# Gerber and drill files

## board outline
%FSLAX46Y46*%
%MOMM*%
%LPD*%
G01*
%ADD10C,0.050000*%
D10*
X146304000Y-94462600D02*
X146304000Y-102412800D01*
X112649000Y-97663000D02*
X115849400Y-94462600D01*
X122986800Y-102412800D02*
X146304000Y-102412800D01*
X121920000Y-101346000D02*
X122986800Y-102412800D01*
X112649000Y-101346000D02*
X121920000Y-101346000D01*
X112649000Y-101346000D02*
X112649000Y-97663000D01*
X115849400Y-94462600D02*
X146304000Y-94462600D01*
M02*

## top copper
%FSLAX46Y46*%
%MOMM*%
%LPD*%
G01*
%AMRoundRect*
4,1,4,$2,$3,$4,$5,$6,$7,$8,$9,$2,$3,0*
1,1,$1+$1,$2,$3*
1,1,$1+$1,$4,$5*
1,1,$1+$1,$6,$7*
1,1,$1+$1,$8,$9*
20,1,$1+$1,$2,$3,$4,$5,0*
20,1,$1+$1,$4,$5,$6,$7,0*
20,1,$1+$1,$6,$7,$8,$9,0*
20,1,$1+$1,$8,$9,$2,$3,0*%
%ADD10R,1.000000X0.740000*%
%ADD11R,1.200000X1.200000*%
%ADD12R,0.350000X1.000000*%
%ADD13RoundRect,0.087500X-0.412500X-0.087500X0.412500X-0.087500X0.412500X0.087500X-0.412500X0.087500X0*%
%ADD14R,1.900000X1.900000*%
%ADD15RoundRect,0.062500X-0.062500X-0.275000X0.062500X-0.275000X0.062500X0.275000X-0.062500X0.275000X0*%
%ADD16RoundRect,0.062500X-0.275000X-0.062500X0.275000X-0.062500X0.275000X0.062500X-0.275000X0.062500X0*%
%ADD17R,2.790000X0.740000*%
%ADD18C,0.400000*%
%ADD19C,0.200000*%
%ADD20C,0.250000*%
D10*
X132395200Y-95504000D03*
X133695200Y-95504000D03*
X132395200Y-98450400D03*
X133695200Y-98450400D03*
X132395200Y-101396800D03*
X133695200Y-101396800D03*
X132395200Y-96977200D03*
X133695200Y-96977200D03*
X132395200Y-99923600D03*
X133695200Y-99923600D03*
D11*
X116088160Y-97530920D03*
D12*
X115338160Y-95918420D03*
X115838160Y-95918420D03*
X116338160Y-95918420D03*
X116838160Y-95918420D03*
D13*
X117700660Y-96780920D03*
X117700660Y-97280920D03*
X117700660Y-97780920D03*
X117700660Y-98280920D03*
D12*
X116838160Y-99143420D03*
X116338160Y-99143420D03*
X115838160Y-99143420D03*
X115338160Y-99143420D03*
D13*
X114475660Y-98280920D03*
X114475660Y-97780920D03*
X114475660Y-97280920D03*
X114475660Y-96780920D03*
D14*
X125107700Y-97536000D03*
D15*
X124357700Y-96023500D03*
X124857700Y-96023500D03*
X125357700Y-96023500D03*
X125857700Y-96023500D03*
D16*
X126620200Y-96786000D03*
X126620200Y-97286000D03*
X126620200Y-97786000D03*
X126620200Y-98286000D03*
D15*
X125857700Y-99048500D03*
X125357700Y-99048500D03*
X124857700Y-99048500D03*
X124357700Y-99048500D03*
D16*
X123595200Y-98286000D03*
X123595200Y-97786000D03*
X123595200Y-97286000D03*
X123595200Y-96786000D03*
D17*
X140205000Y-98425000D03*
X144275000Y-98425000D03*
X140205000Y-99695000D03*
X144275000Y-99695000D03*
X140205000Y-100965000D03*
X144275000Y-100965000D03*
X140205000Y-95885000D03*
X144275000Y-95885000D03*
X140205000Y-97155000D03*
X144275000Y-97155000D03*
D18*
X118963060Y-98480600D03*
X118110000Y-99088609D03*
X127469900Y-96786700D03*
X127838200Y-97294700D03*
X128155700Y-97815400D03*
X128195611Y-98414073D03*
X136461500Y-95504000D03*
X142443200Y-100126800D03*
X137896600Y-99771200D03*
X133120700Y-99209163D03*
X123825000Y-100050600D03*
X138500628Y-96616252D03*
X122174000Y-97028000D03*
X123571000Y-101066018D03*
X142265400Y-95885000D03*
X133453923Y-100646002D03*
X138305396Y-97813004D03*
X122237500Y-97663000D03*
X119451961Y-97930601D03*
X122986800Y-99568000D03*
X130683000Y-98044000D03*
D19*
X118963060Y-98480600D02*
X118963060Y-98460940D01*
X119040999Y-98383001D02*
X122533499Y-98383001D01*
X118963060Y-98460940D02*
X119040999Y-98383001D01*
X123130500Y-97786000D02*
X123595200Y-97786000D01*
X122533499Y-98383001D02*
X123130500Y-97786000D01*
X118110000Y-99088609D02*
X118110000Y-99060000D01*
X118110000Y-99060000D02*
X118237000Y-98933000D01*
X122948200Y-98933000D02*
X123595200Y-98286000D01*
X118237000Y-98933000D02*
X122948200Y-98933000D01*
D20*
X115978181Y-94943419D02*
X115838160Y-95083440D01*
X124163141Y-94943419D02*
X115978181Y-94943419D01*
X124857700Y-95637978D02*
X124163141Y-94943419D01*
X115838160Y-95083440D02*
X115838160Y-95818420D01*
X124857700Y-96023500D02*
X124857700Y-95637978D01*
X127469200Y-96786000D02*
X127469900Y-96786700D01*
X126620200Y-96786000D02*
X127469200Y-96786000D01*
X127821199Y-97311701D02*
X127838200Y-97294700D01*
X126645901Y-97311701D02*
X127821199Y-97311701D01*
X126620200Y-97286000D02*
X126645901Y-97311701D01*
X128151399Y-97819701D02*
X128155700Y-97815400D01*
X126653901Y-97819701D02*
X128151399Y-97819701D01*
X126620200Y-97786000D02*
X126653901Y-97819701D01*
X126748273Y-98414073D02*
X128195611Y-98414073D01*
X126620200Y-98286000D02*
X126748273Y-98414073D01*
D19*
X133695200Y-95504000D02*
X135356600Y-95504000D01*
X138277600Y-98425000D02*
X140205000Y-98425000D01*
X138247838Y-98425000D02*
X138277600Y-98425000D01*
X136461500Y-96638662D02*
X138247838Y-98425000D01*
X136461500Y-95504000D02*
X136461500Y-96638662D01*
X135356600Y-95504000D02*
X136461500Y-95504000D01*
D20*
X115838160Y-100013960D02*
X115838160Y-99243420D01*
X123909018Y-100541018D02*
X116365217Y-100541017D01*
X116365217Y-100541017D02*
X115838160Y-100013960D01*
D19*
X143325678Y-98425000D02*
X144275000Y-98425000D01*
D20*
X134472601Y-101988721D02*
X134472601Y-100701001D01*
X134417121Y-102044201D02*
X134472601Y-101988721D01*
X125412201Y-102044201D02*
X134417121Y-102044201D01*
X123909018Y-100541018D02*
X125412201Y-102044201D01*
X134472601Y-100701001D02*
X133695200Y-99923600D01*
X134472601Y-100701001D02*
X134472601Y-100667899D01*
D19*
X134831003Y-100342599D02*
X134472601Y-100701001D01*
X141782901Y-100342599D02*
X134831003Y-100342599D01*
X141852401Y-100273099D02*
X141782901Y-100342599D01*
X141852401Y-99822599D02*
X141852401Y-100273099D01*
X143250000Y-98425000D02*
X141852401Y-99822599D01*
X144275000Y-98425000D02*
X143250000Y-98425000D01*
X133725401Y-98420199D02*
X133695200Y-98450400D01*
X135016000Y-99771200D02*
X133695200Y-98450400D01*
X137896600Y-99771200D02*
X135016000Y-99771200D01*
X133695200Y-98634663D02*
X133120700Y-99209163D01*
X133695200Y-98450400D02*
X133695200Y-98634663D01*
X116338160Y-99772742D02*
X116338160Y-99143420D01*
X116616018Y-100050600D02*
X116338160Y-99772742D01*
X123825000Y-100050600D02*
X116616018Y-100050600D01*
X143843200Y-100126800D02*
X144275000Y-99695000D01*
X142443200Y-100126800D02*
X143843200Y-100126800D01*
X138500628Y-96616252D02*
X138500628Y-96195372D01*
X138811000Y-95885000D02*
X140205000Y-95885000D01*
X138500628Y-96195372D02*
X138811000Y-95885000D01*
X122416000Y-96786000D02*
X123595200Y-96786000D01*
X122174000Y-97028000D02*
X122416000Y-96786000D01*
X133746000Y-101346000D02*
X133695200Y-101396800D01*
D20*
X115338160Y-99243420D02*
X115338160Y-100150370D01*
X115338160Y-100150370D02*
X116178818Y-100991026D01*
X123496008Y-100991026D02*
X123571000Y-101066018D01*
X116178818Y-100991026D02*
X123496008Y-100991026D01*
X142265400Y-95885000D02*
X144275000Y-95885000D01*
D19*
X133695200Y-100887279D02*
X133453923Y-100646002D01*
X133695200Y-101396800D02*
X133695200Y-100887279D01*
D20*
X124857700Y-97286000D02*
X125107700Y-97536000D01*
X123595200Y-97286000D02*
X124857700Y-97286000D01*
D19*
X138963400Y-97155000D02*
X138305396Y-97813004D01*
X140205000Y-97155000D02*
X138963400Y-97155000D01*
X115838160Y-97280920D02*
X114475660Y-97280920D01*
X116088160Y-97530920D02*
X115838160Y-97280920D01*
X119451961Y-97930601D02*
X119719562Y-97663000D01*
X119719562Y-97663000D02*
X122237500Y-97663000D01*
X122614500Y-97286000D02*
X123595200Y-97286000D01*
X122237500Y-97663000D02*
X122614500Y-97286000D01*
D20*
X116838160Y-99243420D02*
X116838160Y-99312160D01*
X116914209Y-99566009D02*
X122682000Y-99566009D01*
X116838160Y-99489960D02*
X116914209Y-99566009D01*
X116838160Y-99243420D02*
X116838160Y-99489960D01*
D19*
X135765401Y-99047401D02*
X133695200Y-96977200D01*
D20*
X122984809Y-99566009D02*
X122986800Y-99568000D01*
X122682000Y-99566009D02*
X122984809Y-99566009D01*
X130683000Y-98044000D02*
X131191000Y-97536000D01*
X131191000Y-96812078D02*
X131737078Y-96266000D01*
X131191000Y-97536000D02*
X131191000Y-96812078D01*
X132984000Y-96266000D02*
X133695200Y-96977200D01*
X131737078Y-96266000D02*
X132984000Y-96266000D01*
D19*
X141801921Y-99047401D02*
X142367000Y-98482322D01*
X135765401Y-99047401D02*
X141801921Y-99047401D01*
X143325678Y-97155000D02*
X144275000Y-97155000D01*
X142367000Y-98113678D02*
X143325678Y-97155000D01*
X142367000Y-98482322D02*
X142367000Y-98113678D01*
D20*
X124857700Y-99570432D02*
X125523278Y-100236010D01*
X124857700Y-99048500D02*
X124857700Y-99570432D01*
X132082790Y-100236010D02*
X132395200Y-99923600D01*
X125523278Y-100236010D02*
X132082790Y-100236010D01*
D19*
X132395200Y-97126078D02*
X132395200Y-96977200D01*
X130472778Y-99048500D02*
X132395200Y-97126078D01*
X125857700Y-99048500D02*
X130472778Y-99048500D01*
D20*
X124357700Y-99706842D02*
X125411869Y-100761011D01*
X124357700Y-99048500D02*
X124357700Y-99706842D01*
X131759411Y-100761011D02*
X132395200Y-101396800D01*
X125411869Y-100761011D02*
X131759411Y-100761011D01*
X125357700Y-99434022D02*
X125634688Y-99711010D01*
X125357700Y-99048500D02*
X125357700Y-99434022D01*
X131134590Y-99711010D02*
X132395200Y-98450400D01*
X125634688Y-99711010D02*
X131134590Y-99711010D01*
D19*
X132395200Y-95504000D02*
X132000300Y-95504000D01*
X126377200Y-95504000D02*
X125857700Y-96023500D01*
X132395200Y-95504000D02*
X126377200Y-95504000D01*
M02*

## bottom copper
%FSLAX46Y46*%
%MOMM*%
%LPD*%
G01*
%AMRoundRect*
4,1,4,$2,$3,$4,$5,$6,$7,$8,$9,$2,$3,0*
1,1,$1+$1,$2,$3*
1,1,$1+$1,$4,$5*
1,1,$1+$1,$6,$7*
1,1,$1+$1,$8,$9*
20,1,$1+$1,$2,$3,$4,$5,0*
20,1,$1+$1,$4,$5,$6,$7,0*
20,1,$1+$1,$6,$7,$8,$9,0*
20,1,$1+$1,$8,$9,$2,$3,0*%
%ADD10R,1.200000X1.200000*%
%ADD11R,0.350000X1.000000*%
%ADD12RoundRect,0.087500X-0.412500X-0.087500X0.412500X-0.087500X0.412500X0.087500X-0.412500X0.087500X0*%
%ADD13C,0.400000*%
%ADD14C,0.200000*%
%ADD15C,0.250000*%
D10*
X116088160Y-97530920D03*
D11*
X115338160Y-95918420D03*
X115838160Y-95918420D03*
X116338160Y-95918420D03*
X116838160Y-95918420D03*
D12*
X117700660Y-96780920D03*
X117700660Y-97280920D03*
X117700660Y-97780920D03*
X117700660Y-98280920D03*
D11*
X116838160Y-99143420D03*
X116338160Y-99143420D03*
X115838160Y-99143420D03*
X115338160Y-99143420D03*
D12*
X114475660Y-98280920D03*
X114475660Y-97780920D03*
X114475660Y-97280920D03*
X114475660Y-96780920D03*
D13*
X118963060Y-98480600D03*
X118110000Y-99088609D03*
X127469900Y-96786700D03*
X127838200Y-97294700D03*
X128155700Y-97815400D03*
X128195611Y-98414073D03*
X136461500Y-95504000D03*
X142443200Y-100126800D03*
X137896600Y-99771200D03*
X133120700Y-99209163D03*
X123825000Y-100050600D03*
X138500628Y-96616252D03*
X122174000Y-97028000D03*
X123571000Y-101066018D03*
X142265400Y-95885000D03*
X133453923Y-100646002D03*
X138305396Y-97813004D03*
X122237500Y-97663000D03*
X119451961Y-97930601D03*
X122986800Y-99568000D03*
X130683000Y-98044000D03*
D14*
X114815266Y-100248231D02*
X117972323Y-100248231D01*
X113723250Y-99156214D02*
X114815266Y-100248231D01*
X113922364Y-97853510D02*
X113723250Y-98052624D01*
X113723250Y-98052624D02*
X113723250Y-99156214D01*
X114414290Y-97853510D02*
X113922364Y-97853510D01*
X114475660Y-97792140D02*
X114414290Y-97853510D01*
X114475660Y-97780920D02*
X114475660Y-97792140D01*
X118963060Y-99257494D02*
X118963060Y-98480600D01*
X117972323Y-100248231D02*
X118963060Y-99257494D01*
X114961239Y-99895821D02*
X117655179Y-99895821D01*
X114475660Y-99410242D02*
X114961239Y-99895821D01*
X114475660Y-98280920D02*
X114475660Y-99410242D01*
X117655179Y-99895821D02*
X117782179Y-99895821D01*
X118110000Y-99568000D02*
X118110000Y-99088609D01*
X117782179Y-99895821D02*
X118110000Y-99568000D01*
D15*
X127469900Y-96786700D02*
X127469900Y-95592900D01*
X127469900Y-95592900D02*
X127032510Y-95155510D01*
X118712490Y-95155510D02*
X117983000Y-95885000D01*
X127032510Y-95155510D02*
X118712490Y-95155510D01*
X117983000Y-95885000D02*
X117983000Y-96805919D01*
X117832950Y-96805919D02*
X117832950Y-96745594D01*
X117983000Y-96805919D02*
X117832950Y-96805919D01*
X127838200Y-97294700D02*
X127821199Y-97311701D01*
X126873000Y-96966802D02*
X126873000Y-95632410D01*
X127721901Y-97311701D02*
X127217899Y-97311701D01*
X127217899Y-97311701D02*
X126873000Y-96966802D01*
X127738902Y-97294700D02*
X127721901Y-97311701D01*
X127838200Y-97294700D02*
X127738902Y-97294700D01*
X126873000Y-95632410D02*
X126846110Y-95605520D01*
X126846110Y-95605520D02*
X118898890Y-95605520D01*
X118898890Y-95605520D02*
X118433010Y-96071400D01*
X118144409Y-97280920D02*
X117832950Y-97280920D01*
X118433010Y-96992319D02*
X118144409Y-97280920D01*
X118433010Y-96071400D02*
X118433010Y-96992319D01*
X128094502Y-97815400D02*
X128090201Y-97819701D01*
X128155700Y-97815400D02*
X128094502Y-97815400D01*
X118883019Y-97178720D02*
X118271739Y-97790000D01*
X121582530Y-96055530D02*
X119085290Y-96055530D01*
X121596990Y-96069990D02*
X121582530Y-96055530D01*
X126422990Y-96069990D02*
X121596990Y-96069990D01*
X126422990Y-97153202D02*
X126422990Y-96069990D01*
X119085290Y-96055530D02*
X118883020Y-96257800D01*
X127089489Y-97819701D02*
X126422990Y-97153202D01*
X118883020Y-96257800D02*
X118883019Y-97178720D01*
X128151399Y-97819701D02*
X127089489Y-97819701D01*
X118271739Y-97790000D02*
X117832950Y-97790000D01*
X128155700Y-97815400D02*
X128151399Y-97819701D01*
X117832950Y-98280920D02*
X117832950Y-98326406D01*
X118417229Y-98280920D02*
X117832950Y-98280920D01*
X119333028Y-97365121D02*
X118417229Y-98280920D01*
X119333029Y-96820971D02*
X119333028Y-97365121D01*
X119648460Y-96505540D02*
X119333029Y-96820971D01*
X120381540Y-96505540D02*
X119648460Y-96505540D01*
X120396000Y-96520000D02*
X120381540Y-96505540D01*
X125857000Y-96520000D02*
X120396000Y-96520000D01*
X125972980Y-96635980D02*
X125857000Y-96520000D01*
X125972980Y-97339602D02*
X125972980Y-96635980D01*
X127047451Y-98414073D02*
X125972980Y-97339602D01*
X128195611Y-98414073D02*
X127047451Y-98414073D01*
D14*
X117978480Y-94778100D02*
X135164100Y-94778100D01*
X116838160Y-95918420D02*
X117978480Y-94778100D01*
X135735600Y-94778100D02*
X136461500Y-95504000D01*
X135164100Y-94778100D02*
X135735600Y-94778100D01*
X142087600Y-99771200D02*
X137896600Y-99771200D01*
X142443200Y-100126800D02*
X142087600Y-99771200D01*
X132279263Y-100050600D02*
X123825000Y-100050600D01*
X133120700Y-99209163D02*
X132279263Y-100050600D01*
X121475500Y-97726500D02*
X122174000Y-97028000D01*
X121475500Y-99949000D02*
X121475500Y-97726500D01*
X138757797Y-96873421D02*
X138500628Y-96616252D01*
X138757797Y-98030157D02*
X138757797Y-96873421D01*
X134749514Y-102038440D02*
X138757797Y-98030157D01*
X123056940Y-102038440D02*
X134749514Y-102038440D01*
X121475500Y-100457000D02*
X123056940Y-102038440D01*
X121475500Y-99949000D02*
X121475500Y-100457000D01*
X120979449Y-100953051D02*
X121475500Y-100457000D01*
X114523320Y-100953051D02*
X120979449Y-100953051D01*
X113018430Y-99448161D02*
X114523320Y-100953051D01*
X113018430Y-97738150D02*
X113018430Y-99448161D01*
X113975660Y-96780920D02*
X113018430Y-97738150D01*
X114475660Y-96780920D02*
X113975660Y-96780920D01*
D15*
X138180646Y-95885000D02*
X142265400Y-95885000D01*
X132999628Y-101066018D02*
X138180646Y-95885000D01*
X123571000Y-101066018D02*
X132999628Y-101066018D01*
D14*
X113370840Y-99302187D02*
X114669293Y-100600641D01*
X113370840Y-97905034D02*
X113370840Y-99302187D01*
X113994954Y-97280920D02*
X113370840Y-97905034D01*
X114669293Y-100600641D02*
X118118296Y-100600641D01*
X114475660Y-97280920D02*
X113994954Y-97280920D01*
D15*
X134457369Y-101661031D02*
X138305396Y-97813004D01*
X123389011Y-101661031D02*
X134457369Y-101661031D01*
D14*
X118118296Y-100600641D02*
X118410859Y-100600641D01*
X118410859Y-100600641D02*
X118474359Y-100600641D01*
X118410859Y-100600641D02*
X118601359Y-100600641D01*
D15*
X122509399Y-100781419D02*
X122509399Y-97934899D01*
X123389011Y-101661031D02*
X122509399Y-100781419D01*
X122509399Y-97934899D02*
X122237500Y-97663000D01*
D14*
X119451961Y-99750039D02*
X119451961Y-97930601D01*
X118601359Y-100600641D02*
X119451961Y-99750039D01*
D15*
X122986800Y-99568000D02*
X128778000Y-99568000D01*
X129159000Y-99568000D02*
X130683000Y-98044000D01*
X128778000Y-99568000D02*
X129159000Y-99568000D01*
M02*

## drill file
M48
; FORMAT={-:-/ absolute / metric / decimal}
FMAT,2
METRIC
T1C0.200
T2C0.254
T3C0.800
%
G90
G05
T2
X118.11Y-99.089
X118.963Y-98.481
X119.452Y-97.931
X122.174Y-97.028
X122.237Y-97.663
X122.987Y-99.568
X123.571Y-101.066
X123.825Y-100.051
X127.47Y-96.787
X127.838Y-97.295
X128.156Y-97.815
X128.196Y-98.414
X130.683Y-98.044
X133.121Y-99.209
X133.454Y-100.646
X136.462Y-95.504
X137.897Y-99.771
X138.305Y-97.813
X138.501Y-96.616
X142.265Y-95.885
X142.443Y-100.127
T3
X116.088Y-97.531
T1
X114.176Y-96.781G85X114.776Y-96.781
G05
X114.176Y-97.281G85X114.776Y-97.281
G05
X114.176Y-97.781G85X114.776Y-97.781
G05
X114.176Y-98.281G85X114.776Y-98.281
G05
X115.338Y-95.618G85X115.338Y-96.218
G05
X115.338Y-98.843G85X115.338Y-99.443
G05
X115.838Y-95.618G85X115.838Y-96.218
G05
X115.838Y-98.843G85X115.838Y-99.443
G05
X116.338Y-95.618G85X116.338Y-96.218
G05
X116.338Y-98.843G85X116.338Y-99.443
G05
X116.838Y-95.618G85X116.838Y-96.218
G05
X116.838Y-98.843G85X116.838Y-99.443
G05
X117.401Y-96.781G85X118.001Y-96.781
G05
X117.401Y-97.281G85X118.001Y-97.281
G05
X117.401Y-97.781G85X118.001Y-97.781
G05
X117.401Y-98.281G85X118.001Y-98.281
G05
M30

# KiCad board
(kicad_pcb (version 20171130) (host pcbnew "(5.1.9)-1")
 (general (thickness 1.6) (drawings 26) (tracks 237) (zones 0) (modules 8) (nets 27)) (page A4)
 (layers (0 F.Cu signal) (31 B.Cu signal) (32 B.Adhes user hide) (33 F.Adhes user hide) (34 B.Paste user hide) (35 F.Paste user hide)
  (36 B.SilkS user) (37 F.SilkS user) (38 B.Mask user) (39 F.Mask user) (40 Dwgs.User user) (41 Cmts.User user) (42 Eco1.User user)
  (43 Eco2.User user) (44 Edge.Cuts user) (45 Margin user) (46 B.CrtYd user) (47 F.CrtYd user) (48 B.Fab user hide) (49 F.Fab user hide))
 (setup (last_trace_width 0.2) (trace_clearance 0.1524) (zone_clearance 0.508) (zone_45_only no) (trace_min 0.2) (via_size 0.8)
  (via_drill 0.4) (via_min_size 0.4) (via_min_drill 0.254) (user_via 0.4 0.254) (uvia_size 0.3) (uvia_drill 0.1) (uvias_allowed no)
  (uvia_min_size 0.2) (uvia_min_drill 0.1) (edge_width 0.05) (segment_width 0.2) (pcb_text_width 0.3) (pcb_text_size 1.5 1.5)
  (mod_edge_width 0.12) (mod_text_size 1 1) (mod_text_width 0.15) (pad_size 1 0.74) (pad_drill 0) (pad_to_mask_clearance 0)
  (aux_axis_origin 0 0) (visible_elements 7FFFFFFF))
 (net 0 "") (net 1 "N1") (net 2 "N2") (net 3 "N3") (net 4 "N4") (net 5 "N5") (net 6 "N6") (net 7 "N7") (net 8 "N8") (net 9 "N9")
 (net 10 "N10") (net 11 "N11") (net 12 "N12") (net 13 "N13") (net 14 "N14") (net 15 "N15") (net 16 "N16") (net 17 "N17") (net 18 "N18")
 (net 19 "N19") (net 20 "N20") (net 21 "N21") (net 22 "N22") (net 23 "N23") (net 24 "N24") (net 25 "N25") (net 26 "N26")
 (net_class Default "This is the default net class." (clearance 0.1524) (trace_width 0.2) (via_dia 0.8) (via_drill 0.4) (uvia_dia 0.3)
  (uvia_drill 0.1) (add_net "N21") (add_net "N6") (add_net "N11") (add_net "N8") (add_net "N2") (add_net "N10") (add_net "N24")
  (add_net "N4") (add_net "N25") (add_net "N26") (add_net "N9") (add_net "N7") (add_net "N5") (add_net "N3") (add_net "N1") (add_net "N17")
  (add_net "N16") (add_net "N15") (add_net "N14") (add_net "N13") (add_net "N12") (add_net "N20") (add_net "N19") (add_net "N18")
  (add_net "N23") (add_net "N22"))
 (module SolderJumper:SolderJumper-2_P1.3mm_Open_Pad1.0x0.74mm (layer F.Cu) (at 133.0452 95.504)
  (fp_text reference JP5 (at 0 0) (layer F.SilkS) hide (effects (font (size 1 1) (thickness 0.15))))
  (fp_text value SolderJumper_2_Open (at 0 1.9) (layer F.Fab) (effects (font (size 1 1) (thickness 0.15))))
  (pad 1 smd rect (at -0.65 0) (size 1 0.74) (layers F.Cu F.Mask) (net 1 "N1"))
  (pad 2 smd rect (at 0.65 0) (size 1 0.74) (layers F.Cu F.Mask) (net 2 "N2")))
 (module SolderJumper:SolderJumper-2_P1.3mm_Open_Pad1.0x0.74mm (layer F.Cu) (at 133.0452 98.4504)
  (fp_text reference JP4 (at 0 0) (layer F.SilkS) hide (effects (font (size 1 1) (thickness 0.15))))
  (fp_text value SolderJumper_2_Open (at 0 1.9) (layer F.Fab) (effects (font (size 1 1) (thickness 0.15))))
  (pad 1 smd rect (at -0.65 0) (size 1 0.74) (layers F.Cu F.Mask) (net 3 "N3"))
  (pad 2 smd rect (at 0.65 0) (size 1 0.74) (layers F.Cu F.Mask) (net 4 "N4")))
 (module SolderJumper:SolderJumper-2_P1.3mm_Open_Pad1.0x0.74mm (layer F.Cu) (at 133.0452 101.3968)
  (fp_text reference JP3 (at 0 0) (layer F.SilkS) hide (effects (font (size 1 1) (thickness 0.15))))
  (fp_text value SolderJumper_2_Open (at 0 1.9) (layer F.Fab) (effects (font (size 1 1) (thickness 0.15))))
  (pad 1 smd rect (at -0.65 0) (size 1 0.74) (layers F.Cu F.Mask) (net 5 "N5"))
  (pad 2 smd rect (at 0.65 0) (size 1 0.74) (layers F.Cu F.Mask) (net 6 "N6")))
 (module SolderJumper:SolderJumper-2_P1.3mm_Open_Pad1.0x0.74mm (layer F.Cu) (at 133.0452 96.9772)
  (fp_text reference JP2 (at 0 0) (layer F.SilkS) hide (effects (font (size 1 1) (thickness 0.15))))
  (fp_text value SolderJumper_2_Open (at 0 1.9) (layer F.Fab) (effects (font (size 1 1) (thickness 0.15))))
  (pad 1 smd rect (at -0.65 0) (size 1 0.74) (layers F.Cu F.Mask) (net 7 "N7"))
  (pad 2 smd rect (at 0.65 0) (size 1 0.74) (layers F.Cu F.Mask) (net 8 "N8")))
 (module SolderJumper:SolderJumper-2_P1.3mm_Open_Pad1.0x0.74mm (layer F.Cu) (at 133.0452 99.9236)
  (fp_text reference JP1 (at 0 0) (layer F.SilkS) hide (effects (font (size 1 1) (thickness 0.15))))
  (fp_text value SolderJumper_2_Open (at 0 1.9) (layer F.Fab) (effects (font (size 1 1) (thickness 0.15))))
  (pad 1 smd rect (at -0.65 0) (size 1 0.74) (layers F.Cu F.Mask) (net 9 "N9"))
  (pad 2 smd rect (at 0.65 0) (size 1 0.74) (layers F.Cu F.Mask) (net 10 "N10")))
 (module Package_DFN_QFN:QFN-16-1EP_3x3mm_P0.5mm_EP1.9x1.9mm (layer F.Cu) (at 116.08816 97.53092)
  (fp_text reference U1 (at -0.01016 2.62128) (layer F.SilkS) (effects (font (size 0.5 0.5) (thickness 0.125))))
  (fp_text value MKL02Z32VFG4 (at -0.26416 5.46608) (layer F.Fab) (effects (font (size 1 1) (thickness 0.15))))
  (pad "" smd roundrect (at 0.475 0.475) (size 0.77 0.77) (layers F.Paste) (roundrect_rratio 0.25))
  (pad "" smd roundrect (at 0.475 -0.475) (size 0.77 0.77) (layers F.Paste) (roundrect_rratio 0.25))
  (pad "" smd roundrect (at -0.475 0.475) (size 0.77 0.77) (layers F.Paste) (roundrect_rratio 0.25))
  (pad "" smd roundrect (at -0.475 -0.475) (size 0.77 0.77) (layers F.Paste) (roundrect_rratio 0.25))
  (pad 17 thru_hole rect (at 0 0) (size 1.2 1.2) (drill 0.8) (layers *.Cu *.Mask) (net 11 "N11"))
  (pad 16 thru_hole rect (at -0.75 -1.6125) (size 0.35 1) (drill oval 0.2 0.8) (layers *.Cu *.Mask) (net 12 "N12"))
  (pad 15 thru_hole rect (at -0.25 -1.6125) (size 0.35 1) (drill oval 0.2 0.8) (layers *.Cu *.Mask) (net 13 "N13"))
  (pad 14 thru_hole rect (at 0.25 -1.6125) (size 0.35 1) (drill oval 0.2 0.8) (layers *.Cu *.Mask) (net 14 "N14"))
  (pad 13 thru_hole rect (at 0.75 -1.6125) (size 0.35 1) (drill oval 0.2 0.8) (layers *.Cu *.Mask) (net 2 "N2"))
  (pad 12 thru_hole roundrect (at 1.6125 -0.75) (size 1 0.35) (drill oval 0.8 0.2) (layers *.Cu *.Mask) (roundrect_rratio 0.25)
   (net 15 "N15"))
  (pad 11 thru_hole roundrect (at 1.6125 -0.25) (size 1 0.35) (drill oval 0.8 0.2) (layers *.Cu *.Mask) (roundrect_rratio 0.25)
   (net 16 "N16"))
  (pad 10 thru_hole roundrect (at 1.6125 0.25) (size 1 0.35) (drill oval 0.8 0.2) (layers *.Cu *.Mask) (roundrect_rratio 0.25)
   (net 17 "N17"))
  (pad 9 thru_hole roundrect (at 1.6125 0.75) (size 1 0.35) (drill oval 0.8 0.2) (layers *.Cu *.Mask) (roundrect_rratio 0.25) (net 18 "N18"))
  (pad 8 thru_hole rect (at 0.75 1.6125) (size 0.35 1) (drill oval 0.2 0.8) (layers *.Cu *.Mask) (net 8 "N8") (clearance 0.00001))
  (pad 7 thru_hole rect (at 0.25 1.6125) (size 0.35 1) (drill oval 0.2 0.8) (layers *.Cu *.Mask) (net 4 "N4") (clearance 0.000001))
  (pad 6 thru_hole rect (at -0.25 1.6125) (size 0.35 1) (drill oval 0.2 0.8) (layers *.Cu *.Mask) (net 10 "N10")
   (solder_mask_margin 0.000001) (clearance 0.00001))
  (pad 5 thru_hole rect (at -0.75 1.6125) (size 0.35 1) (drill oval 0.2 0.8) (layers *.Cu *.Mask) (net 6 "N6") (clearance 0.00001))
  (pad 4 thru_hole roundrect (at -1.6125 0.75) (size 1 0.35) (drill oval 0.8 0.2) (layers *.Cu *.Mask) (roundrect_rratio 0.25)
   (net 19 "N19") (clearance 0.0001))
  (pad 3 thru_hole roundrect (at -1.6125 0.25) (size 1 0.35) (drill oval 0.8 0.2) (layers *.Cu *.Mask) (roundrect_rratio 0.25)
   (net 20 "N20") (clearance 0.0001))
  (pad 2 thru_hole roundrect (at -1.6125 -0.25) (size 1 0.35) (drill oval 0.8 0.2) (layers *.Cu *.Mask) (roundrect_rratio 0.25)
   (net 11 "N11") (clearance 0.0001))
  (pad 1 thru_hole roundrect (at -1.6125 -0.75) (size 1 0.35) (drill oval 0.8 0.2) (layers *.Cu *.Mask) (roundrect_rratio 0.25)
   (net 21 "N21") (clearance 0.00001)))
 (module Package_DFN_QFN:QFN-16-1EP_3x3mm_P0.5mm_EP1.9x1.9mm (layer F.Cu) (at 125.1077 97.536)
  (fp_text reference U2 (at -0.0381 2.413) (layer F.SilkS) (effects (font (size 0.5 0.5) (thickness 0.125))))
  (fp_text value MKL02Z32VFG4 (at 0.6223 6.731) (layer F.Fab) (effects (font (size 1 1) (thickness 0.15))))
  (pad "" smd roundrect (at 0.475 0.475) (size 0.77 0.77) (layers F.Paste) (roundrect_rratio 0.25))
  (pad "" smd roundrect (at 0.475 -0.475) (size 0.77 0.77) (layers F.Paste) (roundrect_rratio 0.25))
  (pad "" smd roundrect (at -0.475 0.475) (size 0.77 0.77) (layers F.Paste) (roundrect_rratio 0.25))
  (pad "" smd roundrect (at -0.475 -0.475) (size 0.77 0.77) (layers F.Paste) (roundrect_rratio 0.25))
  (pad 17 smd rect (at 0 0) (size 1.9 1.9) (layers F.Cu F.Mask) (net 11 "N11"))
  (pad 16 smd roundrect (at -0.75 -1.5125) (size 0.25 0.675) (layers F.Cu F.Paste F.Mask) (roundrect_rratio 0.25) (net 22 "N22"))
  (pad 15 smd roundrect (at -0.25 -1.5125) (size 0.25 0.675) (layers F.Cu F.Paste F.Mask) (roundrect_rratio 0.25) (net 13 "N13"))
  (pad 14 smd roundrect (at 0.25 -1.5125) (size 0.25 0.675) (layers F.Cu F.Paste F.Mask) (roundrect_rratio 0.25) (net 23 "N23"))
  (pad 13 smd roundrect (at 0.75 -1.5125) (size 0.25 0.675) (layers F.Cu F.Paste F.Mask) (roundrect_rratio 0.25) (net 1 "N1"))
  (pad 12 smd roundrect (at 1.5125 -0.75) (size 0.675 0.25) (layers F.Cu F.Paste F.Mask) (roundrect_rratio 0.25) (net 15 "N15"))
  (pad 11 smd roundrect (at 1.5125 -0.25) (size 0.675 0.25) (layers F.Cu F.Paste F.Mask) (roundrect_rratio 0.25) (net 16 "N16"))
  (pad 10 smd roundrect (at 1.5125 0.25) (size 0.675 0.25) (layers F.Cu F.Paste F.Mask) (roundrect_rratio 0.25) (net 17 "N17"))
  (pad 9 smd roundrect (at 1.5125 0.75) (size 0.675 0.25) (layers F.Cu F.Paste F.Mask) (roundrect_rratio 0.25) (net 18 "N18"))
  (pad 8 smd roundrect (at 0.75 1.5125) (size 0.25 0.675) (layers F.Cu F.Paste F.Mask) (roundrect_rratio 0.25) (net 7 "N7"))
  (pad 7 smd roundrect (at 0.25 1.5125) (size 0.25 0.675) (layers F.Cu F.Paste F.Mask) (roundrect_rratio 0.25) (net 3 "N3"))
  (pad 6 smd roundrect (at -0.25 1.5125) (size 0.25 0.675) (layers F.Cu F.Paste F.Mask) (roundrect_rratio 0.25) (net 9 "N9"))
  (pad 5 smd roundrect (at -0.75 1.5125) (size 0.25 0.675) (layers F.Cu F.Paste F.Mask) (roundrect_rratio 0.25) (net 5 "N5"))
  (pad 4 smd roundrect (at -1.5125 0.75) (size 0.675 0.25) (layers F.Cu F.Paste F.Mask) (roundrect_rratio 0.25) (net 19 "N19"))
  (pad 3 smd roundrect (at -1.5125 0.25) (size 0.675 0.25) (layers F.Cu F.Paste F.Mask) (roundrect_rratio 0.25) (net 20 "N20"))
  (pad 2 smd roundrect (at -1.5125 -0.25) (size 0.675 0.25) (layers F.Cu F.Paste F.Mask) (roundrect_rratio 0.25) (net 11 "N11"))
  (pad 1 smd roundrect (at -1.5125 -0.75) (size 0.675 0.25) (layers F.Cu F.Paste F.Mask) (roundrect_rratio 0.25) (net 21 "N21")))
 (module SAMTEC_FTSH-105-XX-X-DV (layer F.Cu) (at 142.24 98.425 270)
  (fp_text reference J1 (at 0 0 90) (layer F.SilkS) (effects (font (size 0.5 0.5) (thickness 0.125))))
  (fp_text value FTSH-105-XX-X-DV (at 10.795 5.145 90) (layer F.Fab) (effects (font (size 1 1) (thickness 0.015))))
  (pad 05 smd rect (at 0 2.035 270) (size 0.74 2.79) (layers F.Cu F.Paste F.Mask) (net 2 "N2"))
  (pad 06 smd rect (at 0 -2.035 270) (size 0.74 2.79) (layers F.Cu F.Paste F.Mask) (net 10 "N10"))
  (pad 07 smd rect (at 1.27 2.035 270) (size 0.74 2.79) (layers F.Cu F.Paste F.Mask) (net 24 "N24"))
  (pad 08 smd rect (at 1.27 -2.035 270) (size 0.74 2.79) (layers F.Cu F.Paste F.Mask) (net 4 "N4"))
  (pad 09 smd rect (at 2.54 2.035 270) (size 0.74 2.79) (layers F.Cu F.Paste F.Mask) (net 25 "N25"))
  (pad 10 smd rect (at 2.54 -2.035 270) (size 0.74 2.79) (layers F.Cu F.Paste F.Mask) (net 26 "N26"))
  (pad 01 smd rect (at -2.54 2.035 270) (size 0.74 2.79) (layers F.Cu F.Paste F.Mask) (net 21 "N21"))
  (pad 02 smd rect (at -2.54 -2.035 270) (size 0.74 2.79) (layers F.Cu F.Paste F.Mask) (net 6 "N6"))
  (pad 03 smd rect (at -1.27 2.035 270) (size 0.74 2.79) (layers F.Cu F.Paste F.Mask) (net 11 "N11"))
  (pad 04 smd rect (at -1.27 -2.035 270) (size 0.74 2.79) (layers F.Cu F.Paste F.Mask) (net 8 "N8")))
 (gr_line (start 146.304 94.4626) (end 146.304 102.4128) (layer Edge.Cuts) (width 0.05))
 (gr_line (start 112.649 97.663) (end 115.8494 94.4626) (layer Edge.Cuts) (width 0.05))
 (gr_line (start 122.9868 102.4128) (end 146.304 102.4128) (layer Edge.Cuts) (width 0.05))
 (gr_line (start 121.92 101.346) (end 122.9868 102.4128) (layer Edge.Cuts) (width 0.05))
 (gr_line (start 112.649 101.346) (end 121.92 101.346) (layer Edge.Cuts) (width 0.05))
 (gr_line (start 112.649 101.346) (end 112.649 97.663) (layer Edge.Cuts) (width 0.05))
 (gr_line (start 115.8494 94.4626) (end 146.304 94.4626) (layer Edge.Cuts) (width 0.05))
 (segment (start 114.815266 100.248231) (end 117.972323 100.248231) (width 0.2) (layer B.Cu) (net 20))
 (segment (start 113.72325 99.156214) (end 114.815266 100.248231) (width 0.2) (layer B.Cu) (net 20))
 (segment (start 113.922364 97.85351) (end 113.72325 98.052624) (width 0.2) (layer B.Cu) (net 20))
 (segment (start 113.72325 98.052624) (end 113.72325 99.156214) (width 0.2) (layer B.Cu) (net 20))
 (segment (start 114.41429 97.85351) (end 113.922364 97.85351) (width 0.2) (layer B.Cu) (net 20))
 (segment (start 114.47566 97.79214) (end 114.41429 97.85351) (width 0.2) (layer B.Cu) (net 20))
 (segment (start 114.47566 97.78092) (end 114.47566 97.79214) (width 0.2) (layer B.Cu) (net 20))
 (via (at 118.96306 98.4806) (size 0.4) (drill 0.254) (layers F.Cu B.Cu) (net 20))
 (segment (start 118.96306 99.257494) (end 118.96306 98.4806) (width 0.2) (layer B.Cu) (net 20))
 (segment (start 117.972323 100.248231) (end 118.96306 99.257494) (width 0.2) (layer B.Cu) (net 20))
 (segment (start 118.96306 98.4806) (end 118.96306 98.46094) (width 0.2) (layer F.Cu) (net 20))
 (segment (start 119.040999 98.383001) (end 122.533499 98.383001) (width 0.2) (layer F.Cu) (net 20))
 (segment (start 118.96306 98.46094) (end 119.040999 98.383001) (width 0.2) (layer F.Cu) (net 20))
 (segment (start 123.1305 97.786) (end 123.5952 97.786) (width 0.2) (layer F.Cu) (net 20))
 (segment (start 122.533499 98.383001) (end 123.1305 97.786) (width 0.2) (layer F.Cu) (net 20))
 (segment (start 114.961239 99.895821) (end 117.655179 99.895821) (width 0.2) (layer B.Cu) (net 19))
 (segment (start 114.47566 99.410242) (end 114.961239 99.895821) (width 0.2) (layer B.Cu) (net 19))
 (segment (start 114.47566 98.28092) (end 114.47566 99.410242) (width 0.2) (layer B.Cu) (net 19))
 (segment (start 117.655179 99.895821) (end 117.782179 99.895821) (width 0.2) (layer B.Cu) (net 19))
 (via (at 118.11 99.088609) (size 0.4) (drill 0.254) (layers F.Cu B.Cu) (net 19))
 (segment (start 118.11 99.568) (end 118.11 99.088609) (width 0.2) (layer B.Cu) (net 19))
 (segment (start 117.782179 99.895821) (end 118.11 99.568) (width 0.2) (layer B.Cu) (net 19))
 (segment (start 118.11 99.088609) (end 118.11 99.06) (width 0.2) (layer F.Cu) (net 19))
 (segment (start 118.11 99.06) (end 118.237 98.933) (width 0.2) (layer F.Cu) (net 19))
 (segment (start 122.9482 98.933) (end 123.5952 98.286) (width 0.2) (layer F.Cu) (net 19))
 (segment (start 118.237 98.933) (end 122.9482 98.933) (width 0.2) (layer F.Cu) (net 19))
 (segment (start 115.978181 94.943419) (end 115.83816 95.08344) (width 0.25) (layer F.Cu) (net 13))
 (segment (start 124.163141 94.943419) (end 115.978181 94.943419) (width 0.25) (layer F.Cu) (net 13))
 (segment (start 124.8577 95.637978) (end 124.163141 94.943419) (width 0.25) (layer F.Cu) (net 13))
 (segment (start 115.83816 95.08344) (end 115.83816 95.81842) (width 0.25) (layer F.Cu) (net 13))
 (segment (start 124.8577 96.0235) (end 124.8577 95.637978) (width 0.25) (layer F.Cu) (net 13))
 (via (at 127.4699 96.7867) (size 0.4) (drill 0.254) (layers F.Cu B.Cu) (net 15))
 (segment (start 127.4692 96.786) (end 127.4699 96.7867) (width 0.25) (layer F.Cu) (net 15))
 (segment (start 126.6202 96.786) (end 127.4692 96.786) (width 0.25) (layer F.Cu) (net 15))
 (segment (start 127.4699 96.7867) (end 127.4699 95.5929) (width 0.25) (layer B.Cu) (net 15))
 (segment (start 127.4699 95.5929) (end 127.03251 95.15551) (width 0.25) (layer B.Cu) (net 15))
 (segment (start 118.71249 95.15551) (end 117.983 95.885) (width 0.25) (layer B.Cu) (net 15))
 (segment (start 127.03251 95.15551) (end 118.71249 95.15551) (width 0.25) (layer B.Cu) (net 15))
 (segment (start 117.983 95.885) (end 117.983 96.805919) (width 0.25) (layer B.Cu) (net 15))
 (segment (start 117.83295 96.805919) (end 117.83295 96.745594) (width 0.25) (layer B.Cu) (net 15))
 (segment (start 117.983 96.805919) (end 117.83295 96.805919) (width 0.25) (layer B.Cu) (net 15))
 (segment (start 127.821199 97.311701) (end 127.8382 97.2947) (width 0.25) (layer F.Cu) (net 16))
 (segment (start 126.645901 97.311701) (end 127.821199 97.311701) (width 0.25) (layer F.Cu) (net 16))
 (via (at 127.8382 97.2947) (size 0.4) (drill 0.254) (layers F.Cu B.Cu) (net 16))
 (segment (start 126.6202 97.286) (end 126.645901 97.311701) (width 0.25) (layer F.Cu) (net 16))
 (segment (start 127.8382 97.2947) (end 127.821199 97.311701) (width 0.25) (layer B.Cu) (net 16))
 (segment (start 126.873 96.966802) (end 126.873 95.63241) (width 0.25) (layer B.Cu) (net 16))
 (segment (start 127.721901 97.311701) (end 127.217899 97.311701) (width 0.25) (layer B.Cu) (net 16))
 (segment (start 127.217899 97.311701) (end 126.873 96.966802) (width 0.25) (layer B.Cu) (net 16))
 (segment (start 127.738902 97.2947) (end 127.721901 97.311701) (width 0.25) (layer B.Cu) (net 16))
 (segment (start 127.8382 97.2947) (end 127.738902 97.2947) (width 0.25) (layer B.Cu) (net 16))
 (segment (start 126.873 95.63241) (end 126.84611 95.60552) (width 0.25) (layer B.Cu) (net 16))
 (segment (start 126.84611 95.60552) (end 118.89889 95.60552) (width 0.25) (layer B.Cu) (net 16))
 (segment (start 118.89889 95.60552) (end 118.43301 96.0714) (width 0.25) (layer B.Cu) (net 16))
 (segment (start 118.144409 97.28092) (end 117.83295 97.28092) (width 0.25) (layer B.Cu) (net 16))
 (segment (start 118.43301 96.992319) (end 118.144409 97.28092) (width 0.25) (layer B.Cu) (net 16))
 (segment (start 118.43301 96.0714) (end 118.43301 96.992319) (width 0.25) (layer B.Cu) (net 16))
 (via (at 128.1557 97.8154) (size 0.4) (drill 0.254) (layers F.Cu B.Cu) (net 17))
 (segment (start 128.151399 97.819701) (end 128.1557 97.8154) (width 0.25) (layer F.Cu) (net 17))
 (segment (start 126.653901 97.819701) (end 128.151399 97.819701) (width 0.25) (layer F.Cu) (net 17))
 (segment (start 126.6202 97.786) (end 126.653901 97.819701) (width 0.25) (layer F.Cu) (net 17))
 (segment (start 128.094502 97.8154) (end 128.090201 97.819701) (width 0.25) (layer B.Cu) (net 17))
 (segment (start 128.1557 97.8154) (end 128.094502 97.8154) (width 0.25) (layer B.Cu) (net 17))
 (segment (start 118.883019 97.17872) (end 118.271739 97.79) (width 0.25) (layer B.Cu) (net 17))
 (segment (start 121.58253 96.05553) (end 119.08529 96.05553) (width 0.25) (layer B.Cu) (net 17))
 (segment (start 121.59699 96.06999) (end 121.58253 96.05553) (width 0.25) (layer B.Cu) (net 17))
 (segment (start 126.42299 96.06999) (end 121.59699 96.06999) (width 0.25) (layer B.Cu) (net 17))
 (segment (start 126.42299 97.153202) (end 126.42299 96.06999) (width 0.25) (layer B.Cu) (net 17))
 (segment (start 119.08529 96.05553) (end 118.88302 96.2578) (width 0.25) (layer B.Cu) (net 17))
 (segment (start 127.089489 97.819701) (end 126.42299 97.153202) (width 0.25) (layer B.Cu) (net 17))
 (segment (start 118.88302 96.2578) (end 118.883019 97.17872) (width 0.25) (layer B.Cu) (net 17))
 (segment (start 128.151399 97.819701) (end 127.089489 97.819701) (width 0.25) (layer B.Cu) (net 17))
 (segment (start 118.271739 97.79) (end 117.83295 97.79) (width 0.25) (layer B.Cu) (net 17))
 (segment (start 128.1557 97.8154) (end 128.151399 97.819701) (width 0.25) (layer B.Cu) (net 17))
 (via (at 128.195611 98.414073) (size 0.4) (drill 0.254) (layers F.Cu B.Cu) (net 18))
 (segment (start 126.748273 98.414073) (end 128.195611 98.414073) (width 0.25) (layer F.Cu) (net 18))
 (segment (start 126.6202 98.286) (end 126.748273 98.414073) (width 0.25) (layer F.Cu) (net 18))
 (segment (start 117.83295 98.28092) (end 117.83295 98.326406) (width 0.25) (layer B.Cu) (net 18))
 (segment (start 118.417229 98.28092) (end 117.83295 98.28092) (width 0.25) (layer B.Cu) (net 18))
 (segment (start 119.333028 97.365121) (end 118.417229 98.28092) (width 0.25) (layer B.Cu) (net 18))
 (segment (start 119.333029 96.820971) (end 119.333028 97.365121) (width 0.25) (layer B.Cu) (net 18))
 (segment (start 119.64846 96.50554) (end 119.333029 96.820971) (width 0.25) (layer B.Cu) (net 18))
 (segment (start 120.38154 96.50554) (end 119.64846 96.50554) (width 0.25) (layer B.Cu) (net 18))
 (segment (start 120.396 96.52) (end 120.38154 96.50554) (width 0.25) (layer B.Cu) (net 18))
 (segment (start 125.857 96.52) (end 120.396 96.52) (width 0.25) (layer B.Cu) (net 18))
 (segment (start 125.97298 96.63598) (end 125.857 96.52) (width 0.25) (layer B.Cu) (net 18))
 (segment (start 125.97298 97.339602) (end 125.97298 96.63598) (width 0.25) (layer B.Cu) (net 18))
 (segment (start 127.047451 98.414073) (end 125.97298 97.339602) (width 0.25) (layer B.Cu) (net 18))
 (segment (start 128.195611 98.414073) (end 127.047451 98.414073) (width 0.25) (layer B.Cu) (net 18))
 (segment (start 117.97848 94.7781) (end 135.1641 94.7781) (width 0.2) (layer B.Cu) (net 2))
 (segment (start 116.83816 95.91842) (end 117.97848 94.7781) (width 0.2) (layer B.Cu) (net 2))
 (segment (start 133.6952 95.504) (end 135.3566 95.504) (width 0.2) (layer F.Cu) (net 2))
 (segment (start 138.2776 98.425) (end 140.205 98.425) (width 0.2) (layer F.Cu) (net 2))
 (via (at 136.4615 95.504) (size 0.4) (drill 0.254) (layers F.Cu B.Cu) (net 2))
 (segment (start 135.7356 94.7781) (end 136.4615 95.504) (width 0.2) (layer B.Cu) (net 2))
 (segment (start 135.1641 94.7781) (end 135.7356 94.7781) (width 0.2) (layer B.Cu) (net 2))
 (segment (start 138.247838 98.425) (end 138.2776 98.425) (width 0.2) (layer F.Cu) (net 2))
 (segment (start 136.4615 96.638662) (end 138.247838 98.425) (width 0.2) (layer F.Cu) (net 2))
 (segment (start 136.4615 95.504) (end 136.4615 96.638662) (width 0.2) (layer F.Cu) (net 2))
 (segment (start 135.3566 95.504) (end 136.4615 95.504) (width 0.2) (layer F.Cu) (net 2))
 (segment (start 115.83816 100.01396) (end 115.83816 99.24342) (width 0.25) (layer F.Cu) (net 10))
 (segment (start 123.909018 100.541018) (end 116.365217 100.541017) (width 0.25) (layer F.Cu) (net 10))
 (segment (start 116.365217 100.541017) (end 115.83816 100.01396) (width 0.25) (layer F.Cu) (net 10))
 (segment (start 143.325678 98.425) (end 144.275 98.425) (width 0.2) (layer F.Cu) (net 10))
 (segment (start 134.472601 101.988721) (end 134.472601 100.701001) (width 0.25) (layer F.Cu) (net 10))
 (segment (start 134.417121 102.044201) (end 134.472601 101.988721) (width 0.25) (layer F.Cu) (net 10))
 (segment (start 125.412201 102.044201) (end 134.417121 102.044201) (width 0.25) (layer F.Cu) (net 10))
 (segment (start 123.909018 100.541018) (end 125.412201 102.044201) (width 0.25) (layer F.Cu) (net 10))
 (segment (start 134.472601 100.701001) (end 133.6952 99.9236) (width 0.25) (layer F.Cu) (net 10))
 (segment (start 134.472601 100.701001) (end 134.472601 100.667899) (width 0.25) (layer F.Cu) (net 10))
 (segment (start 134.831003 100.342599) (end 134.472601 100.701001) (width 0.2) (layer F.Cu) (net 10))
 (segment (start 141.782901 100.342599) (end 134.831003 100.342599) (width 0.2) (layer F.Cu) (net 10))
 (segment (start 141.852401 100.273099) (end 141.782901 100.342599) (width 0.2) (layer F.Cu) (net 10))
 (segment (start 141.852401 99.822599) (end 141.852401 100.273099) (width 0.2) (layer F.Cu) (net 10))
 (segment (start 143.25 98.425) (end 141.852401 99.822599) (width 0.2) (layer F.Cu) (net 10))
 (segment (start 144.275 98.425) (end 143.25 98.425) (width 0.2) (layer F.Cu) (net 10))
 (segment (start 133.725401 98.420199) (end 133.6952 98.4504) (width 0.2) (layer F.Cu) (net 4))
 (via (at 142.4432 100.1268) (size 0.4) (drill 0.254) (layers F.Cu B.Cu) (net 4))
 (via (at 137.8966 99.7712) (size 0.4) (drill 0.254) (layers F.Cu B.Cu) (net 4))
 (segment (start 142.0876 99.7712) (end 137.8966 99.7712) (width 0.2) (layer B.Cu) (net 4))
 (segment (start 142.4432 100.1268) (end 142.0876 99.7712) (width 0.2) (layer B.Cu) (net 4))
 (segment (start 135.016 99.7712) (end 133.6952 98.4504) (width 0.2) (layer F.Cu) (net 4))
 (segment (start 137.8966 99.7712) (end 135.016 99.7712) (width 0.2) (layer F.Cu) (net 4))
 (via (at 133.1207 99.209163) (size 0.4) (drill 0.254) (layers F.Cu B.Cu) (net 4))
 (segment (start 133.6952 98.634663) (end 133.1207 99.209163) (width 0.2) (layer F.Cu) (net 4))
 (segment (start 133.6952 98.4504) (end 133.6952 98.634663) (width 0.2) (layer F.Cu) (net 4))
 (via (at 123.825 100.0506) (size 0.4) (drill 0.254) (layers F.Cu B.Cu) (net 4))
 (segment (start 132.279263 100.0506) (end 123.825 100.0506) (width 0.2) (layer B.Cu) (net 4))
 (segment (start 133.1207 99.209163) (end 132.279263 100.0506) (width 0.2) (layer B.Cu) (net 4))
 (segment (start 116.33816 99.772742) (end 116.33816 99.14342) (width 0.2) (layer F.Cu) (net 4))
 (segment (start 116.616018 100.0506) (end 116.33816 99.772742) (width 0.2) (layer F.Cu) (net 4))
 (segment (start 123.825 100.0506) (end 116.616018 100.0506) (width 0.2) (layer F.Cu) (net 4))
 (segment (start 143.8432 100.1268) (end 144.275 99.695) (width 0.2) (layer F.Cu) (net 4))
 (segment (start 142.4432 100.1268) (end 143.8432 100.1268) (width 0.2) (layer F.Cu) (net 4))
 (via (at 138.500628 96.616252) (size 0.4) (drill 0.254) (layers F.Cu B.Cu) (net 21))
 (segment (start 138.500628 96.616252) (end 138.500628 96.195372) (width 0.2) (layer F.Cu) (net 21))
 (segment (start 138.811 95.885) (end 140.205 95.885) (width 0.2) (layer F.Cu) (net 21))
 (segment (start 138.500628 96.195372) (end 138.811 95.885) (width 0.2) (layer F.Cu) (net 21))
 (via (at 122.174 97.028) (size 0.4) (drill 0.254) (layers F.Cu B.Cu) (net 21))
 (segment (start 121.4755 97.7265) (end 122.174 97.028) (width 0.2) (layer B.Cu) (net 21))
 (segment (start 121.4755 99.949) (end 121.4755 97.7265) (width 0.2) (layer B.Cu) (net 21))
 (segment (start 122.416 96.786) (end 123.5952 96.786) (width 0.2) (layer F.Cu) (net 21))
 (segment (start 122.174 97.028) (end 122.416 96.786) (width 0.2) (layer F.Cu) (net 21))
 (segment (start 138.757797 96.873421) (end 138.500628 96.616252) (width 0.2) (layer B.Cu) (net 21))
 (segment (start 138.757797 98.030157) (end 138.757797 96.873421) (width 0.2) (layer B.Cu) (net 21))
 (segment (start 134.749514 102.03844) (end 138.757797 98.030157) (width 0.2) (layer B.Cu) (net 21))
 (segment (start 123.05694 102.03844) (end 134.749514 102.03844) (width 0.2) (layer B.Cu) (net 21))
 (segment (start 121.4755 100.457) (end 123.05694 102.03844) (width 0.2) (layer B.Cu) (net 21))
 (segment (start 121.4755 99.949) (end 121.4755 100.457) (width 0.2) (layer B.Cu) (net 21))
 (segment (start 120.979449 100.953051) (end 121.4755 100.457) (width 0.2) (layer B.Cu) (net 21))
 (segment (start 114.52332 100.953051) (end 120.979449 100.953051) (width 0.2) (layer B.Cu) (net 21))
 (segment (start 113.01843 99.448161) (end 114.52332 100.953051) (width 0.2) (layer B.Cu) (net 21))
 (segment (start 113.01843 97.73815) (end 113.01843 99.448161) (width 0.2) (layer B.Cu) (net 21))
 (segment (start 113.97566 96.78092) (end 113.01843 97.73815) (width 0.2) (layer B.Cu) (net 21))
 (segment (start 114.47566 96.78092) (end 113.97566 96.78092) (width 0.2) (layer B.Cu) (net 21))
 (segment (start 133.746 101.346) (end 133.6952 101.3968) (width 0.2) (layer F.Cu) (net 6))
 (segment (start 115.33816 99.24342) (end 115.33816 100.15037) (width 0.25) (layer F.Cu) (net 6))
 (segment (start 115.33816 100.15037) (end 116.178818 100.991026) (width 0.25) (layer F.Cu) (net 6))
 (segment (start 123.496008 100.991026) (end 123.571 101.066018) (width 0.25) (layer F.Cu) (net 6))
 (via (at 123.571 101.066018) (size 0.4) (drill 0.254) (layers F.Cu B.Cu) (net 6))
 (segment (start 116.178818 100.991026) (end 123.496008 100.991026) (width 0.25) (layer F.Cu) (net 6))
 (via (at 142.2654 95.885) (size 0.4) (drill 0.254) (layers F.Cu B.Cu) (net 6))
 (segment (start 138.180646 95.885) (end 142.2654 95.885) (width 0.25) (layer B.Cu) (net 6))
 (segment (start 132.999628 101.066018) (end 138.180646 95.885) (width 0.25) (layer B.Cu) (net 6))
 (segment (start 123.571 101.066018) (end 132.999628 101.066018) (width 0.25) (layer B.Cu) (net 6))
 (segment (start 142.2654 95.885) (end 144.275 95.885) (width 0.25) (layer F.Cu) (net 6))
 (segment (start 133.6952 100.887279) (end 133.453923 100.646002) (width 0.2) (layer F.Cu) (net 6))
 (via (at 133.453923 100.646002) (size 0.4) (drill 0.254) (layers F.Cu B.Cu) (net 6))
 (segment (start 133.6952 101.3968) (end 133.6952 100.887279) (width 0.2) (layer F.Cu) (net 6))
 (segment (start 124.8577 97.286) (end 125.1077 97.536) (width 0.25) (layer F.Cu) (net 11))
 (segment (start 123.5952 97.286) (end 124.8577 97.286) (width 0.25) (layer F.Cu) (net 11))
 (segment (start 113.37084 99.302187) (end 114.669293 100.600641) (width 0.2) (layer B.Cu) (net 11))
 (segment (start 113.37084 97.905034) (end 113.37084 99.302187) (width 0.2) (layer B.Cu) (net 11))
 (segment (start 113.994954 97.28092) (end 113.37084 97.905034) (width 0.2) (layer B.Cu) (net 11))
 (segment (start 114.669293 100.600641) (end 118.118296 100.600641) (width 0.2) (layer B.Cu) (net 11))
 (segment (start 114.47566 97.28092) (end 113.994954 97.28092) (width 0.2) (layer B.Cu) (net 11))
 (segment (start 138.9634 97.155) (end 138.305396 97.813004) (width 0.2) (layer F.Cu) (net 11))
 (via (at 138.305396 97.813004) (size 0.4) (drill 0.254) (layers F.Cu B.Cu) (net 11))
 (segment (start 140.205 97.155) (end 138.9634 97.155) (width 0.2) (layer F.Cu) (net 11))
 (segment (start 134.457369 101.661031) (end 138.305396 97.813004) (width 0.25) (layer B.Cu) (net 11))
 (segment (start 123.389011 101.661031) (end 134.457369 101.661031) (width 0.25) (layer B.Cu) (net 11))
 (segment (start 115.83816 97.28092) (end 114.47566 97.28092) (width 0.2) (layer F.Cu) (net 11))
 (segment (start 116.08816 97.53092) (end 115.83816 97.28092) (width 0.2) (layer F.Cu) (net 11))
 (segment (start 118.118296 100.600641) (end 118.410859 100.600641) (width 0.2) (layer B.Cu) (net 11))
 (segment (start 118.410859 100.600641) (end 118.474359 100.600641) (width 0.2) (layer B.Cu) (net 11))
 (segment (start 118.410859 100.600641) (end 118.601359 100.600641) (width 0.2) (layer B.Cu) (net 11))
 (segment (start 122.509399 100.781419) (end 122.509399 97.934899) (width 0.25) (layer B.Cu) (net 11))
 (segment (start 123.389011 101.661031) (end 122.509399 100.781419) (width 0.25) (layer B.Cu) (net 11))
 (via (at 122.2375 97.663) (size 0.4) (drill 0.254) (layers F.Cu B.Cu) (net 11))
 (segment (start 122.509399 97.934899) (end 122.2375 97.663) (width 0.25) (layer B.Cu) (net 11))
 (via (at 119.451961 97.930601) (size 0.4) (drill 0.254) (layers F.Cu B.Cu) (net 11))
 (segment (start 119.451961 99.750039) (end 119.451961 97.930601) (width 0.2) (layer B.Cu) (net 11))
 (segment (start 118.601359 100.600641) (end 119.451961 99.750039) (width 0.2) (layer B.Cu) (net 11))
 (segment (start 119.451961 97.930601) (end 119.719562 97.663) (width 0.2) (layer F.Cu) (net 11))
 (segment (start 119.719562 97.663) (end 122.2375 97.663) (width 0.2) (layer F.Cu) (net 11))
 (segment (start 122.6145 97.286) (end 123.5952 97.286) (width 0.2) (layer F.Cu) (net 11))
 (segment (start 122.2375 97.663) (end 122.6145 97.286) (width 0.2) (layer F.Cu) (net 11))
 (segment (start 116.83816 99.24342) (end 116.83816 99.31216) (width 0.25) (layer F.Cu) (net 8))
 (segment (start 116.914209 99.566009) (end 122.682 99.566009) (width 0.25) (layer F.Cu) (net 8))
 (segment (start 116.83816 99.48996) (end 116.914209 99.566009) (width 0.25) (layer F.Cu) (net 8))
 (segment (start 116.83816 99.24342) (end 116.83816 99.48996) (width 0.25) (layer F.Cu) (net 8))
 (segment (start 135.765401 99.047401) (end 133.6952 96.9772) (width 0.2) (layer F.Cu) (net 8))
 (via (at 122.9868 99.568) (size 0.4) (drill 0.254) (layers F.Cu B.Cu) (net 8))
 (segment (start 122.984809 99.566009) (end 122.9868 99.568) (width 0.25) (layer F.Cu) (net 8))
 (segment (start 122.682 99.566009) (end 122.984809 99.566009) (width 0.25) (layer F.Cu) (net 8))
 (segment (start 122.9868 99.568) (end 128.778 99.568) (width 0.25) (layer B.Cu) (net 8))
 (segment (start 129.159 99.568) (end 130.683 98.044) (width 0.25) (layer B.Cu) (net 8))
 (via (at 130.683 98.044) (size 0.4) (drill 0.254) (layers F.Cu B.Cu) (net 8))
 (segment (start 128.778 99.568) (end 129.159 99.568) (width 0.25) (layer B.Cu) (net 8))
 (segment (start 130.683 98.044) (end 131.191 97.536) (width 0.25) (layer F.Cu) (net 8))
 (segment (start 131.191 96.812078) (end 131.737078 96.266) (width 0.25) (layer F.Cu) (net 8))
 (segment (start 131.191 97.536) (end 131.191 96.812078) (width 0.25) (layer F.Cu) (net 8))
 (segment (start 132.984 96.266) (end 133.6952 96.9772) (width 0.25) (layer F.Cu) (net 8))
 (segment (start 131.737078 96.266) (end 132.984 96.266) (width 0.25) (layer F.Cu) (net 8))
 (segment (start 141.801921 99.047401) (end 142.367 98.482322) (width 0.2) (layer F.Cu) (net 8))
 (segment (start 135.765401 99.047401) (end 141.801921 99.047401) (width 0.2) (layer F.Cu) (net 8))
 (segment (start 143.325678 97.155) (end 144.275 97.155) (width 0.2) (layer F.Cu) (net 8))
 (segment (start 142.367 98.113678) (end 143.325678 97.155) (width 0.2) (layer F.Cu) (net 8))
 (segment (start 142.367 98.482322) (end 142.367 98.113678) (width 0.2) (layer F.Cu) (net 8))
 (segment (start 124.8577 99.570432) (end 125.523278 100.23601) (width 0.25) (layer F.Cu) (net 9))
 (segment (start 124.8577 99.0485) (end 124.8577 99.570432) (width 0.25) (layer F.Cu) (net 9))
 (segment (start 132.08279 100.23601) (end 132.3952 99.9236) (width 0.25) (layer F.Cu) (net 9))
 (segment (start 125.523278 100.23601) (end 132.08279 100.23601) (width 0.25) (layer F.Cu) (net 9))
 (segment (start 132.3952 97.126078) (end 132.3952 96.9772) (width 0.2) (layer F.Cu) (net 7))
 (segment (start 130.472778 99.0485) (end 132.3952 97.126078) (width 0.2) (layer F.Cu) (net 7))
 (segment (start 125.8577 99.0485) (end 130.472778 99.0485) (width 0.2) (layer F.Cu) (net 7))
 (segment (start 124.3577 99.706842) (end 125.411869 100.761011) (width 0.25) (layer F.Cu) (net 5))
 (segment (start 124.3577 99.0485) (end 124.3577 99.706842) (width 0.25) (layer F.Cu) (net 5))
 (segment (start 131.759411 100.761011) (end 132.3952 101.3968) (width 0.25) (layer F.Cu) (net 5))
 (segment (start 125.411869 100.761011) (end 131.759411 100.761011) (width 0.25) (layer F.Cu) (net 5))
 (segment (start 125.3577 99.434022) (end 125.634688 99.71101) (width 0.25) (layer F.Cu) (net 3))
 (segment (start 125.3577 99.0485) (end 125.3577 99.434022) (width 0.25) (layer F.Cu) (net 3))
 (segment (start 131.13459 99.71101) (end 132.3952 98.4504) (width 0.25) (layer F.Cu) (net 3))
 (segment (start 125.634688 99.71101) (end 131.13459 99.71101) (width 0.25) (layer F.Cu) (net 3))
 (segment (start 132.3952 95.504) (end 132.0003 95.504) (width 0.2) (layer F.Cu) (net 1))
 (segment (start 126.3772 95.504) (end 125.8577 96.0235) (width 0.2) (layer F.Cu) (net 1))
 (segment (start 132.3952 95.504) (end 126.3772 95.504) (width 0.2) (layer F.Cu) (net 1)))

